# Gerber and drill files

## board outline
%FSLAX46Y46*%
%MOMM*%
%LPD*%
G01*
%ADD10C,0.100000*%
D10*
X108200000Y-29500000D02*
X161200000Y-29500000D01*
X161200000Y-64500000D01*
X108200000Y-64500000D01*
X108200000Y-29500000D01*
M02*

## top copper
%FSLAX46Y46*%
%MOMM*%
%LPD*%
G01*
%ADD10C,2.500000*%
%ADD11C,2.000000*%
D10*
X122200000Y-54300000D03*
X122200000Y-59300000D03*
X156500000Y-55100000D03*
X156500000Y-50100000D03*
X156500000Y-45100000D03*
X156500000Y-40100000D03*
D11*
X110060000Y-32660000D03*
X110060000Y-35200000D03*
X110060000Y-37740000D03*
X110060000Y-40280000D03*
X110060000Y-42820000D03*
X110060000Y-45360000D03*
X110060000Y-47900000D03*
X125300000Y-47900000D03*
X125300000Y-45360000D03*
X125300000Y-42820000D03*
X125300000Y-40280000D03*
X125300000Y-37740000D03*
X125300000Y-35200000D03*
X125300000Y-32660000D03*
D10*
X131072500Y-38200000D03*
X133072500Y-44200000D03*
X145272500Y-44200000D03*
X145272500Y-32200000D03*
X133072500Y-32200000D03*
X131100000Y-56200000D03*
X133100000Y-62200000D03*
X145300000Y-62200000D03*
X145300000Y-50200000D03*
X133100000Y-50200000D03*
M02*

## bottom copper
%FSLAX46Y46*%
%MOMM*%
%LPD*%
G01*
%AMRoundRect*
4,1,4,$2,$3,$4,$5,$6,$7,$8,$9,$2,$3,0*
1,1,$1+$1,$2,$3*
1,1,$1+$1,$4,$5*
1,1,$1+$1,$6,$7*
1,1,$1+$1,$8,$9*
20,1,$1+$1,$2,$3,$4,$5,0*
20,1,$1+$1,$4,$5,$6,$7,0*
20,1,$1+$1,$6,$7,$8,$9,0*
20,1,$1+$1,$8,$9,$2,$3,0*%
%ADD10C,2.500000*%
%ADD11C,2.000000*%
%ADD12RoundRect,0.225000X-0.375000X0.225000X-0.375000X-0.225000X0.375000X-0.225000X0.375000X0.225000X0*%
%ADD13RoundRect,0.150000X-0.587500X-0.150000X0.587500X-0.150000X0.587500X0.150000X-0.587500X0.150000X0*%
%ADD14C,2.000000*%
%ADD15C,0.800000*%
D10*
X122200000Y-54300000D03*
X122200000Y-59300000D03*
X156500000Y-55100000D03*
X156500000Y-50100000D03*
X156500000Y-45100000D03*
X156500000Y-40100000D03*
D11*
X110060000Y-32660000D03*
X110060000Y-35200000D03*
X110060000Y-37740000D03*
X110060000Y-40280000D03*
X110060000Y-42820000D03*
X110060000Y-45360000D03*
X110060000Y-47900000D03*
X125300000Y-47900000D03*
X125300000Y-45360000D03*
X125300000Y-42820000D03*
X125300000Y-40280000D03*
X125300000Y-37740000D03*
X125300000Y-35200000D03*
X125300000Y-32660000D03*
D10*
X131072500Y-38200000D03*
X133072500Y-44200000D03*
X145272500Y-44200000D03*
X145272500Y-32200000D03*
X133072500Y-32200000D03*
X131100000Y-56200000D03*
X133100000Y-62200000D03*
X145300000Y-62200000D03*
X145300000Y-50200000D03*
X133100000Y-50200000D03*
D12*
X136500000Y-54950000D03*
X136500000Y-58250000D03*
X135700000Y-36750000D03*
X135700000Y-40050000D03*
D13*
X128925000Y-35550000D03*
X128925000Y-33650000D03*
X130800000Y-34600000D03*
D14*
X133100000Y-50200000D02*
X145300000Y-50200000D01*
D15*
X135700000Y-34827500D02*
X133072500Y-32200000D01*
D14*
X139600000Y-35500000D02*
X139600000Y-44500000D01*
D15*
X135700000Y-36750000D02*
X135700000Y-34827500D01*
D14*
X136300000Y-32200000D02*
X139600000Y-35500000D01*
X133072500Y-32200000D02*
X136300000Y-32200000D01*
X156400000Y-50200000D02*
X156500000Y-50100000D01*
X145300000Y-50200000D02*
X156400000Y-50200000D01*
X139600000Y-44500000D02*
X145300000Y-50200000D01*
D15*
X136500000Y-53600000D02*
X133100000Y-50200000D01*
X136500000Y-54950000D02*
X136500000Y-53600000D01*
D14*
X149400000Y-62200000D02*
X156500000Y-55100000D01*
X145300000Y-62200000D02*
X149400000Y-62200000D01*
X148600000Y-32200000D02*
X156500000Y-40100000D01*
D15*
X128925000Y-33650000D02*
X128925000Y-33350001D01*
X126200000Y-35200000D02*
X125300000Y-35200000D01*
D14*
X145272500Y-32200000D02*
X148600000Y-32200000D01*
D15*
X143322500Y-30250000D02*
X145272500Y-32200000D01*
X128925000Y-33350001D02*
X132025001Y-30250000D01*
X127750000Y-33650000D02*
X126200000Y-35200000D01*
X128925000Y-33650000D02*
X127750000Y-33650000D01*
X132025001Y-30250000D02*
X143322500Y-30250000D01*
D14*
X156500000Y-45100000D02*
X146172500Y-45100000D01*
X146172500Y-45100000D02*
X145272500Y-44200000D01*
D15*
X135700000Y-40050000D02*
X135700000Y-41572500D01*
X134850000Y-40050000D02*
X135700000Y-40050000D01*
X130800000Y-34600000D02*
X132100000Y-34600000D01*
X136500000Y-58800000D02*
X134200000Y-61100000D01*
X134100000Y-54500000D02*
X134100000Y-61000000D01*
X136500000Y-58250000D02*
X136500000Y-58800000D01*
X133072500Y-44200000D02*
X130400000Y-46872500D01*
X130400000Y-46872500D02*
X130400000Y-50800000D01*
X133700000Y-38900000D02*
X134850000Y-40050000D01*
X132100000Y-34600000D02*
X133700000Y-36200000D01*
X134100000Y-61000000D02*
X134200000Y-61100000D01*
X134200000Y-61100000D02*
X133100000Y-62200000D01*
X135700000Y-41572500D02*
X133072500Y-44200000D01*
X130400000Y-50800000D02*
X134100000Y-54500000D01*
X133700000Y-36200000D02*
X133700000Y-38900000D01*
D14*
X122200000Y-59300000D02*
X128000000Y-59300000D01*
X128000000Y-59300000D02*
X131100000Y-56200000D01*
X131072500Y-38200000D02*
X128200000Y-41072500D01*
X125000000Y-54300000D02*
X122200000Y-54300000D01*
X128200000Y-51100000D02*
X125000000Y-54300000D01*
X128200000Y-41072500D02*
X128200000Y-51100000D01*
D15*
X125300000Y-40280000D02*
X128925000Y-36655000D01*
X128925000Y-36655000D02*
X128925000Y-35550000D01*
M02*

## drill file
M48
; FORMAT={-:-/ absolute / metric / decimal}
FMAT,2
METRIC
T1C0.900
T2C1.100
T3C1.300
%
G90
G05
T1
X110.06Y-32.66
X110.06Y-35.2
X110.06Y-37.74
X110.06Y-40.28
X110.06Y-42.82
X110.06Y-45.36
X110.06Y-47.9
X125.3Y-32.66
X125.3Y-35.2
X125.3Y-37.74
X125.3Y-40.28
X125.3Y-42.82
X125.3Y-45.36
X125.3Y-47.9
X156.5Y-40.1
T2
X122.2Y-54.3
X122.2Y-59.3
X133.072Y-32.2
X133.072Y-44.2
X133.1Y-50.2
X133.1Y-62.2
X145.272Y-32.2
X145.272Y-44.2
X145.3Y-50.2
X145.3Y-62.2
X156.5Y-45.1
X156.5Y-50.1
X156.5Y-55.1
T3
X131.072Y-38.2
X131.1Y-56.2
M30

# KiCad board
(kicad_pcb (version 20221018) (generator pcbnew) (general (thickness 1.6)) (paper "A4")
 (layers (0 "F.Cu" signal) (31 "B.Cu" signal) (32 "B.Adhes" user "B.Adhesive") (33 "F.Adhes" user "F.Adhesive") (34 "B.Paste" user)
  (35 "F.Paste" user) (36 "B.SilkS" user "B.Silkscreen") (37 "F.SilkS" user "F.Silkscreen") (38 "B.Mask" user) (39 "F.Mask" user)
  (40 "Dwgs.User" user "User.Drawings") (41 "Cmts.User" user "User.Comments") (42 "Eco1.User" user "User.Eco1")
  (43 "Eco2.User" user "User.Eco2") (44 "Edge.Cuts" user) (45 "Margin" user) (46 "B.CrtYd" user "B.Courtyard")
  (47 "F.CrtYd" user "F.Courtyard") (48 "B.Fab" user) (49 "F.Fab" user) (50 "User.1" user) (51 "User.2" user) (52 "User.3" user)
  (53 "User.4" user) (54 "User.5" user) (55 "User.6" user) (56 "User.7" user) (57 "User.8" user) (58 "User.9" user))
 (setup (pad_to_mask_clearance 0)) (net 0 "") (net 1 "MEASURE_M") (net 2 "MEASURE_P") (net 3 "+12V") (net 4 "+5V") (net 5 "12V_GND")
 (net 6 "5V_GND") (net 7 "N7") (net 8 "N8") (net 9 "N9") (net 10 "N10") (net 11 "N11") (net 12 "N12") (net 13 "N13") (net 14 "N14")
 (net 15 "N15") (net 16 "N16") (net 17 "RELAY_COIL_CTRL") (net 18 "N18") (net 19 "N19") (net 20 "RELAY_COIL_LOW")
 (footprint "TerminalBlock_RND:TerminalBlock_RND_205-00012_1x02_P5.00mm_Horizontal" (layer "F.Cu") (at 122.2 54.3 -90)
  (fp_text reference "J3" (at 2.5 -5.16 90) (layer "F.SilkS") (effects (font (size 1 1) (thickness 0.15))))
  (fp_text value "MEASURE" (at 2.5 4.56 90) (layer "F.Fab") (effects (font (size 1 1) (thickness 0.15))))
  (pad "1" thru_hole circle (at 0 0 270) (size 2.5 2.5) (drill 1.1) (layers "*.Cu" "*.Mask") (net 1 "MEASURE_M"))
  (pad "2" thru_hole circle (at 5 0 270) (size 2.5 2.5) (drill 1.1) (layers "*.Cu" "*.Mask") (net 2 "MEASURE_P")))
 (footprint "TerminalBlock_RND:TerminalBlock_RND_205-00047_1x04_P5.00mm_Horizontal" (layer "F.Cu") (at 156.5 55.1 90)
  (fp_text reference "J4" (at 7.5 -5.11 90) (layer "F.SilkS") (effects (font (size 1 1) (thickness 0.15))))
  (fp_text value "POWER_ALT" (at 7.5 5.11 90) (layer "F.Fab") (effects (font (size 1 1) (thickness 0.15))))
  (pad "1" thru_hole circle (at 0 0 90) (size 2.5 2.5) (drill 1.1) (layers "*.Cu" "*.Mask") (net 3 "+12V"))
  (pad "2" thru_hole circle (at 5 0 90) (size 2.5 2.5) (drill 1.1) (layers "*.Cu" "*.Mask") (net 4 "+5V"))
  (pad "3" thru_hole circle (at 10 0 90) (size 2.5 2.5) (drill 1.1) (layers "*.Cu" "*.Mask") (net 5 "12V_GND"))
  (pad "4" thru_hole circle (at 15 0 90) (size 2.5 2.5) (drill 0.9) (layers "*.Cu" "*.Mask") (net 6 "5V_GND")))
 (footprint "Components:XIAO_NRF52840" (layer "F.Cu") (at 117.68 32.66)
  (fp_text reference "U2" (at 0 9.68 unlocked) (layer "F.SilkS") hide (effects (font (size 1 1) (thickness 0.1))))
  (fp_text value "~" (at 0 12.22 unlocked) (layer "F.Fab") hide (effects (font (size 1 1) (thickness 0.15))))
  (pad "1" thru_hole circle (at -7.62 0) (size 2 2) (drill 0.9) (layers "*.Cu" "*.Mask") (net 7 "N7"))
  (pad "2" thru_hole circle (at -7.62 2.54) (size 2 2) (drill 0.9) (layers "*.Cu" "*.Mask") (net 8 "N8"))
  (pad "3" thru_hole circle (at -7.62 5.08) (size 2 2) (drill 0.9) (layers "*.Cu" "*.Mask") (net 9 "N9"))
  (pad "4" thru_hole circle (at -7.62 7.62) (size 2 2) (drill 0.9) (layers "*.Cu" "*.Mask") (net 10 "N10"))
  (pad "5" thru_hole circle (at -7.62 10.16) (size 2 2) (drill 0.9) (layers "*.Cu" "*.Mask") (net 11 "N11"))
  (pad "6" thru_hole circle (at -7.62 12.7) (size 2 2) (drill 0.9) (layers "*.Cu" "*.Mask") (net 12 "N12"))
  (pad "7" thru_hole circle (at -7.62 15.24) (size 2 2) (drill 0.9) (layers "*.Cu" "*.Mask") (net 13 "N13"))
  (pad "8" thru_hole circle (at 7.62 15.24) (size 2 2) (drill 0.9) (layers "*.Cu" "*.Mask") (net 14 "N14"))
  (pad "9" thru_hole circle (at 7.62 12.7) (size 2 2) (drill 0.9) (layers "*.Cu" "*.Mask") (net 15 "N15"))
  (pad "10" thru_hole circle (at 7.62 10.16) (size 2 2) (drill 0.9) (layers "*.Cu" "*.Mask") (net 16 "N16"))
  (pad "11" thru_hole circle (at 7.62 7.62) (size 2 2) (drill 0.9) (layers "*.Cu" "*.Mask") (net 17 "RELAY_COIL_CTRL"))
  (pad "12" thru_hole circle (at 7.62 5.08) (size 2 2) (drill 0.9) (layers "*.Cu" "*.Mask") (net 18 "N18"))
  (pad "13" thru_hole circle (at 7.62 2.54) (size 2 2) (drill 0.9) (layers "*.Cu" "*.Mask") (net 6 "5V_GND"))
  (pad "14" thru_hole circle (at 7.62 0) (size 2 2) (drill 0.9) (layers "*.Cu" "*.Mask") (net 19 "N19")))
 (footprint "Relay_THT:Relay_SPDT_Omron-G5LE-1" (layer "F.Cu") (at 131.0725 38.2 90)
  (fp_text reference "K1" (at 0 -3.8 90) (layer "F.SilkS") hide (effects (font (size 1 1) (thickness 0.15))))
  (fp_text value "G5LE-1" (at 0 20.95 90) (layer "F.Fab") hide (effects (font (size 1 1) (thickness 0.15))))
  (pad "1" thru_hole circle (at 0 0 90) (size 2.5 2.5) (drill 1.3) (layers "*.Cu" "*.Mask") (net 1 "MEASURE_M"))
  (pad "2" thru_hole circle (at -6 2 90) (size 2.5 2.5) (drill 1.1) (layers "*.Cu" "*.Mask") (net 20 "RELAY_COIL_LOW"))
  (pad "3" thru_hole circle (at -6 14.2 90) (size 2.5 2.5) (drill 1.1) (layers "*.Cu" "*.Mask") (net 5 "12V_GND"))
  (pad "4" thru_hole circle (at 6 14.2 90) (size 2.5 2.5) (drill 1.1) (layers "*.Cu" "*.Mask") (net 6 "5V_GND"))
  (pad "5" thru_hole circle (at 6 2 90) (size 2.5 2.5) (drill 1.1) (layers "*.Cu" "*.Mask") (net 4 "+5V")))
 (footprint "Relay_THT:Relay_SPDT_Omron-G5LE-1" (layer "F.Cu") (at 131.1 56.2 90)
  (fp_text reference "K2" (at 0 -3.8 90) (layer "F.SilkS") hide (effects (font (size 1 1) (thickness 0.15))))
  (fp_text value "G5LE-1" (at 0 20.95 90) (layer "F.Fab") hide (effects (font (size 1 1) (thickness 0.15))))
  (pad "1" thru_hole circle (at 0 0 90) (size 2.5 2.5) (drill 1.3) (layers "*.Cu" "*.Mask") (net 2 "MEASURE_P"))
  (pad "2" thru_hole circle (at -6 2 90) (size 2.5 2.5) (drill 1.1) (layers "*.Cu" "*.Mask") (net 20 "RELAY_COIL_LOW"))
  (pad "3" thru_hole circle (at -6 14.2 90) (size 2.5 2.5) (drill 1.1) (layers "*.Cu" "*.Mask") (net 3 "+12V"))
  (pad "4" thru_hole circle (at 6 14.2 90) (size 2.5 2.5) (drill 1.1) (layers "*.Cu" "*.Mask") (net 4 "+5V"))
  (pad "5" thru_hole circle (at 6 2 90) (size 2.5 2.5) (drill 1.1) (layers "*.Cu" "*.Mask") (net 4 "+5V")))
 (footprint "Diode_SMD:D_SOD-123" (layer "B.Cu") (at 136.5 56.6 -90)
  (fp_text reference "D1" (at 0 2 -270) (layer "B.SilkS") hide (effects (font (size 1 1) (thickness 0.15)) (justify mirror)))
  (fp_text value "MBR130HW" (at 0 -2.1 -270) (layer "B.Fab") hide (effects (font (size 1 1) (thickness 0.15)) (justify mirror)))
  (pad "1" smd roundrect (at -1.65 0 270) (size 0.9 1.2) (layers "B.Cu" "B.Paste" "B.Mask") (roundrect_rratio 0.25) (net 4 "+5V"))
  (pad "2" smd roundrect (at 1.65 0 270) (size 0.9 1.2) (layers "B.Cu" "B.Paste" "B.Mask") (roundrect_rratio 0.25) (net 20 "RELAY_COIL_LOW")))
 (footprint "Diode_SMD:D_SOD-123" (layer "B.Cu") (at 135.7 38.4 -90)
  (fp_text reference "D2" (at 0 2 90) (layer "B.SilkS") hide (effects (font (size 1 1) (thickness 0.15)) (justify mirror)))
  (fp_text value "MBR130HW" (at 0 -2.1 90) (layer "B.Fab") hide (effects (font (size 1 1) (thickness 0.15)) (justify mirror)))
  (pad "1" smd roundrect (at -1.65 0 270) (size 0.9 1.2) (layers "B.Cu" "B.Paste" "B.Mask") (roundrect_rratio 0.25) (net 4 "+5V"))
  (pad "2" smd roundrect (at 1.65 0 270) (size 0.9 1.2) (layers "B.Cu" "B.Paste" "B.Mask") (roundrect_rratio 0.25) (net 20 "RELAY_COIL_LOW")))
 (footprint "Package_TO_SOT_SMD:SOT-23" (layer "B.Cu") (at 129.8625 34.6)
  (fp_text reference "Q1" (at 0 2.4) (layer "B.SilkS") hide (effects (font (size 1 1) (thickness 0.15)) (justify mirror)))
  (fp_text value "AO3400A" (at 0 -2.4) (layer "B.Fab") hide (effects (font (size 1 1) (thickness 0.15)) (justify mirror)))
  (pad "1" smd roundrect (at -0.9375 0.95) (size 1.475 0.6) (layers "B.Cu" "B.Paste" "B.Mask") (roundrect_rratio 0.25)
   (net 17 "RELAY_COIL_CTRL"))
  (pad "2" smd roundrect (at -0.9375 -0.95) (size 1.475 0.6) (layers "B.Cu" "B.Paste" "B.Mask") (roundrect_rratio 0.25) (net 6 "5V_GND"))
  (pad "3" smd roundrect (at 0.9375 0) (size 1.475 0.6) (layers "B.Cu" "B.Paste" "B.Mask") (roundrect_rratio 0.25) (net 20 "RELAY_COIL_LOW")))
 (gr_rect (start 108.2 29.5) (end 161.2 64.5) (stroke (width 0.1) (type default)) (fill none) (layer "Edge.Cuts"))
 (segment (start 133.1 50.2) (end 145.3 50.2) (width 2) (layer "B.Cu") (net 4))
 (segment (start 135.7 34.8275) (end 133.0725 32.2) (width 0.8) (layer "B.Cu") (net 4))
 (segment (start 139.6 35.5) (end 139.6 44.5) (width 2) (layer "B.Cu") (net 4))
 (segment (start 135.7 36.75) (end 135.7 34.8275) (width 0.8) (layer "B.Cu") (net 4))
 (segment (start 136.3 32.2) (end 139.6 35.5) (width 2) (layer "B.Cu") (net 4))
 (segment (start 133.0725 32.2) (end 136.3 32.2) (width 2) (layer "B.Cu") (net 4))
 (segment (start 156.4 50.2) (end 156.5 50.1) (width 2) (layer "B.Cu") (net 4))
 (segment (start 145.3 50.2) (end 156.4 50.2) (width 2) (layer "B.Cu") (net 4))
 (segment (start 139.6 44.5) (end 145.3 50.2) (width 2) (layer "B.Cu") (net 4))
 (segment (start 136.5 53.6) (end 133.1 50.2) (width 0.8) (layer "B.Cu") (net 4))
 (segment (start 136.5 54.95) (end 136.5 53.6) (width 0.8) (layer "B.Cu") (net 4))
 (segment (start 149.4 62.2) (end 156.5 55.1) (width 2) (layer "B.Cu") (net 3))
 (segment (start 145.3 62.2) (end 149.4 62.2) (width 2) (layer "B.Cu") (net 3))
 (segment (start 148.6 32.2) (end 156.5 40.1) (width 2) (layer "B.Cu") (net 6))
 (segment (start 128.925 33.65) (end 128.925 33.350001) (width 0.8) (layer "B.Cu") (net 6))
 (segment (start 126.2 35.2) (end 125.3 35.2) (width 0.8) (layer "B.Cu") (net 6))
 (segment (start 145.2725 32.2) (end 148.6 32.2) (width 2) (layer "B.Cu") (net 6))
 (segment (start 143.3225 30.25) (end 145.2725 32.2) (width 0.8) (layer "B.Cu") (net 6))
 (segment (start 128.925 33.350001) (end 132.025001 30.25) (width 0.8) (layer "B.Cu") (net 6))
 (segment (start 127.75 33.65) (end 126.2 35.2) (width 0.8) (layer "B.Cu") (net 6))
 (segment (start 128.925 33.65) (end 127.75 33.65) (width 0.8) (layer "B.Cu") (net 6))
 (segment (start 132.025001 30.25) (end 143.3225 30.25) (width 0.8) (layer "B.Cu") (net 6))
 (segment (start 156.5 45.1) (end 146.1725 45.1) (width 2) (layer "B.Cu") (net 5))
 (segment (start 146.1725 45.1) (end 145.2725 44.2) (width 2) (layer "B.Cu") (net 5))
 (segment (start 135.7 40.05) (end 135.7 41.5725) (width 0.8) (layer "B.Cu") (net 20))
 (segment (start 134.85 40.05) (end 135.7 40.05) (width 0.8) (layer "B.Cu") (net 20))
 (segment (start 130.8 34.6) (end 132.1 34.6) (width 0.8) (layer "B.Cu") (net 20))
 (segment (start 136.5 58.8) (end 134.2 61.1) (width 0.8) (layer "B.Cu") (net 20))
 (segment (start 134.1 54.5) (end 134.1 61) (width 0.8) (layer "B.Cu") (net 20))
 (segment (start 136.5 58.25) (end 136.5 58.8) (width 0.8) (layer "B.Cu") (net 20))
 (segment (start 133.0725 44.2) (end 130.4 46.8725) (width 0.8) (layer "B.Cu") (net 20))
 (segment (start 130.4 46.8725) (end 130.4 50.8) (width 0.8) (layer "B.Cu") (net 20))
 (segment (start 133.7 38.9) (end 134.85 40.05) (width 0.8) (layer "B.Cu") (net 20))
 (segment (start 132.1 34.6) (end 133.7 36.2) (width 0.8) (layer "B.Cu") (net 20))
 (segment (start 134.1 61) (end 134.2 61.1) (width 0.8) (layer "B.Cu") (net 20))
 (segment (start 134.2 61.1) (end 133.1 62.2) (width 0.8) (layer "B.Cu") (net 20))
 (segment (start 135.7 41.5725) (end 133.0725 44.2) (width 0.8) (layer "B.Cu") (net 20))
 (segment (start 130.4 50.8) (end 134.1 54.5) (width 0.8) (layer "B.Cu") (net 20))
 (segment (start 133.7 36.2) (end 133.7 38.9) (width 0.8) (layer "B.Cu") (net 20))
 (segment (start 122.2 59.3) (end 128 59.3) (width 2) (layer "B.Cu") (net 2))
 (segment (start 128 59.3) (end 131.1 56.2) (width 2) (layer "B.Cu") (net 2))
 (segment (start 131.0725 38.2) (end 128.2 41.0725) (width 2) (layer "B.Cu") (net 1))
 (segment (start 125 54.3) (end 122.2 54.3) (width 2) (layer "B.Cu") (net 1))
 (segment (start 128.2 51.1) (end 125 54.3) (width 2) (layer "B.Cu") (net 1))
 (segment (start 128.2 41.0725) (end 128.2 51.1) (width 2) (layer "B.Cu") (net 1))
 (segment (start 125.3 40.28) (end 128.925 36.655) (width 0.8) (layer "B.Cu") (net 17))
 (segment (start 128.925 36.655) (end 128.925 35.55) (width 0.8) (layer "B.Cu") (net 17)))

